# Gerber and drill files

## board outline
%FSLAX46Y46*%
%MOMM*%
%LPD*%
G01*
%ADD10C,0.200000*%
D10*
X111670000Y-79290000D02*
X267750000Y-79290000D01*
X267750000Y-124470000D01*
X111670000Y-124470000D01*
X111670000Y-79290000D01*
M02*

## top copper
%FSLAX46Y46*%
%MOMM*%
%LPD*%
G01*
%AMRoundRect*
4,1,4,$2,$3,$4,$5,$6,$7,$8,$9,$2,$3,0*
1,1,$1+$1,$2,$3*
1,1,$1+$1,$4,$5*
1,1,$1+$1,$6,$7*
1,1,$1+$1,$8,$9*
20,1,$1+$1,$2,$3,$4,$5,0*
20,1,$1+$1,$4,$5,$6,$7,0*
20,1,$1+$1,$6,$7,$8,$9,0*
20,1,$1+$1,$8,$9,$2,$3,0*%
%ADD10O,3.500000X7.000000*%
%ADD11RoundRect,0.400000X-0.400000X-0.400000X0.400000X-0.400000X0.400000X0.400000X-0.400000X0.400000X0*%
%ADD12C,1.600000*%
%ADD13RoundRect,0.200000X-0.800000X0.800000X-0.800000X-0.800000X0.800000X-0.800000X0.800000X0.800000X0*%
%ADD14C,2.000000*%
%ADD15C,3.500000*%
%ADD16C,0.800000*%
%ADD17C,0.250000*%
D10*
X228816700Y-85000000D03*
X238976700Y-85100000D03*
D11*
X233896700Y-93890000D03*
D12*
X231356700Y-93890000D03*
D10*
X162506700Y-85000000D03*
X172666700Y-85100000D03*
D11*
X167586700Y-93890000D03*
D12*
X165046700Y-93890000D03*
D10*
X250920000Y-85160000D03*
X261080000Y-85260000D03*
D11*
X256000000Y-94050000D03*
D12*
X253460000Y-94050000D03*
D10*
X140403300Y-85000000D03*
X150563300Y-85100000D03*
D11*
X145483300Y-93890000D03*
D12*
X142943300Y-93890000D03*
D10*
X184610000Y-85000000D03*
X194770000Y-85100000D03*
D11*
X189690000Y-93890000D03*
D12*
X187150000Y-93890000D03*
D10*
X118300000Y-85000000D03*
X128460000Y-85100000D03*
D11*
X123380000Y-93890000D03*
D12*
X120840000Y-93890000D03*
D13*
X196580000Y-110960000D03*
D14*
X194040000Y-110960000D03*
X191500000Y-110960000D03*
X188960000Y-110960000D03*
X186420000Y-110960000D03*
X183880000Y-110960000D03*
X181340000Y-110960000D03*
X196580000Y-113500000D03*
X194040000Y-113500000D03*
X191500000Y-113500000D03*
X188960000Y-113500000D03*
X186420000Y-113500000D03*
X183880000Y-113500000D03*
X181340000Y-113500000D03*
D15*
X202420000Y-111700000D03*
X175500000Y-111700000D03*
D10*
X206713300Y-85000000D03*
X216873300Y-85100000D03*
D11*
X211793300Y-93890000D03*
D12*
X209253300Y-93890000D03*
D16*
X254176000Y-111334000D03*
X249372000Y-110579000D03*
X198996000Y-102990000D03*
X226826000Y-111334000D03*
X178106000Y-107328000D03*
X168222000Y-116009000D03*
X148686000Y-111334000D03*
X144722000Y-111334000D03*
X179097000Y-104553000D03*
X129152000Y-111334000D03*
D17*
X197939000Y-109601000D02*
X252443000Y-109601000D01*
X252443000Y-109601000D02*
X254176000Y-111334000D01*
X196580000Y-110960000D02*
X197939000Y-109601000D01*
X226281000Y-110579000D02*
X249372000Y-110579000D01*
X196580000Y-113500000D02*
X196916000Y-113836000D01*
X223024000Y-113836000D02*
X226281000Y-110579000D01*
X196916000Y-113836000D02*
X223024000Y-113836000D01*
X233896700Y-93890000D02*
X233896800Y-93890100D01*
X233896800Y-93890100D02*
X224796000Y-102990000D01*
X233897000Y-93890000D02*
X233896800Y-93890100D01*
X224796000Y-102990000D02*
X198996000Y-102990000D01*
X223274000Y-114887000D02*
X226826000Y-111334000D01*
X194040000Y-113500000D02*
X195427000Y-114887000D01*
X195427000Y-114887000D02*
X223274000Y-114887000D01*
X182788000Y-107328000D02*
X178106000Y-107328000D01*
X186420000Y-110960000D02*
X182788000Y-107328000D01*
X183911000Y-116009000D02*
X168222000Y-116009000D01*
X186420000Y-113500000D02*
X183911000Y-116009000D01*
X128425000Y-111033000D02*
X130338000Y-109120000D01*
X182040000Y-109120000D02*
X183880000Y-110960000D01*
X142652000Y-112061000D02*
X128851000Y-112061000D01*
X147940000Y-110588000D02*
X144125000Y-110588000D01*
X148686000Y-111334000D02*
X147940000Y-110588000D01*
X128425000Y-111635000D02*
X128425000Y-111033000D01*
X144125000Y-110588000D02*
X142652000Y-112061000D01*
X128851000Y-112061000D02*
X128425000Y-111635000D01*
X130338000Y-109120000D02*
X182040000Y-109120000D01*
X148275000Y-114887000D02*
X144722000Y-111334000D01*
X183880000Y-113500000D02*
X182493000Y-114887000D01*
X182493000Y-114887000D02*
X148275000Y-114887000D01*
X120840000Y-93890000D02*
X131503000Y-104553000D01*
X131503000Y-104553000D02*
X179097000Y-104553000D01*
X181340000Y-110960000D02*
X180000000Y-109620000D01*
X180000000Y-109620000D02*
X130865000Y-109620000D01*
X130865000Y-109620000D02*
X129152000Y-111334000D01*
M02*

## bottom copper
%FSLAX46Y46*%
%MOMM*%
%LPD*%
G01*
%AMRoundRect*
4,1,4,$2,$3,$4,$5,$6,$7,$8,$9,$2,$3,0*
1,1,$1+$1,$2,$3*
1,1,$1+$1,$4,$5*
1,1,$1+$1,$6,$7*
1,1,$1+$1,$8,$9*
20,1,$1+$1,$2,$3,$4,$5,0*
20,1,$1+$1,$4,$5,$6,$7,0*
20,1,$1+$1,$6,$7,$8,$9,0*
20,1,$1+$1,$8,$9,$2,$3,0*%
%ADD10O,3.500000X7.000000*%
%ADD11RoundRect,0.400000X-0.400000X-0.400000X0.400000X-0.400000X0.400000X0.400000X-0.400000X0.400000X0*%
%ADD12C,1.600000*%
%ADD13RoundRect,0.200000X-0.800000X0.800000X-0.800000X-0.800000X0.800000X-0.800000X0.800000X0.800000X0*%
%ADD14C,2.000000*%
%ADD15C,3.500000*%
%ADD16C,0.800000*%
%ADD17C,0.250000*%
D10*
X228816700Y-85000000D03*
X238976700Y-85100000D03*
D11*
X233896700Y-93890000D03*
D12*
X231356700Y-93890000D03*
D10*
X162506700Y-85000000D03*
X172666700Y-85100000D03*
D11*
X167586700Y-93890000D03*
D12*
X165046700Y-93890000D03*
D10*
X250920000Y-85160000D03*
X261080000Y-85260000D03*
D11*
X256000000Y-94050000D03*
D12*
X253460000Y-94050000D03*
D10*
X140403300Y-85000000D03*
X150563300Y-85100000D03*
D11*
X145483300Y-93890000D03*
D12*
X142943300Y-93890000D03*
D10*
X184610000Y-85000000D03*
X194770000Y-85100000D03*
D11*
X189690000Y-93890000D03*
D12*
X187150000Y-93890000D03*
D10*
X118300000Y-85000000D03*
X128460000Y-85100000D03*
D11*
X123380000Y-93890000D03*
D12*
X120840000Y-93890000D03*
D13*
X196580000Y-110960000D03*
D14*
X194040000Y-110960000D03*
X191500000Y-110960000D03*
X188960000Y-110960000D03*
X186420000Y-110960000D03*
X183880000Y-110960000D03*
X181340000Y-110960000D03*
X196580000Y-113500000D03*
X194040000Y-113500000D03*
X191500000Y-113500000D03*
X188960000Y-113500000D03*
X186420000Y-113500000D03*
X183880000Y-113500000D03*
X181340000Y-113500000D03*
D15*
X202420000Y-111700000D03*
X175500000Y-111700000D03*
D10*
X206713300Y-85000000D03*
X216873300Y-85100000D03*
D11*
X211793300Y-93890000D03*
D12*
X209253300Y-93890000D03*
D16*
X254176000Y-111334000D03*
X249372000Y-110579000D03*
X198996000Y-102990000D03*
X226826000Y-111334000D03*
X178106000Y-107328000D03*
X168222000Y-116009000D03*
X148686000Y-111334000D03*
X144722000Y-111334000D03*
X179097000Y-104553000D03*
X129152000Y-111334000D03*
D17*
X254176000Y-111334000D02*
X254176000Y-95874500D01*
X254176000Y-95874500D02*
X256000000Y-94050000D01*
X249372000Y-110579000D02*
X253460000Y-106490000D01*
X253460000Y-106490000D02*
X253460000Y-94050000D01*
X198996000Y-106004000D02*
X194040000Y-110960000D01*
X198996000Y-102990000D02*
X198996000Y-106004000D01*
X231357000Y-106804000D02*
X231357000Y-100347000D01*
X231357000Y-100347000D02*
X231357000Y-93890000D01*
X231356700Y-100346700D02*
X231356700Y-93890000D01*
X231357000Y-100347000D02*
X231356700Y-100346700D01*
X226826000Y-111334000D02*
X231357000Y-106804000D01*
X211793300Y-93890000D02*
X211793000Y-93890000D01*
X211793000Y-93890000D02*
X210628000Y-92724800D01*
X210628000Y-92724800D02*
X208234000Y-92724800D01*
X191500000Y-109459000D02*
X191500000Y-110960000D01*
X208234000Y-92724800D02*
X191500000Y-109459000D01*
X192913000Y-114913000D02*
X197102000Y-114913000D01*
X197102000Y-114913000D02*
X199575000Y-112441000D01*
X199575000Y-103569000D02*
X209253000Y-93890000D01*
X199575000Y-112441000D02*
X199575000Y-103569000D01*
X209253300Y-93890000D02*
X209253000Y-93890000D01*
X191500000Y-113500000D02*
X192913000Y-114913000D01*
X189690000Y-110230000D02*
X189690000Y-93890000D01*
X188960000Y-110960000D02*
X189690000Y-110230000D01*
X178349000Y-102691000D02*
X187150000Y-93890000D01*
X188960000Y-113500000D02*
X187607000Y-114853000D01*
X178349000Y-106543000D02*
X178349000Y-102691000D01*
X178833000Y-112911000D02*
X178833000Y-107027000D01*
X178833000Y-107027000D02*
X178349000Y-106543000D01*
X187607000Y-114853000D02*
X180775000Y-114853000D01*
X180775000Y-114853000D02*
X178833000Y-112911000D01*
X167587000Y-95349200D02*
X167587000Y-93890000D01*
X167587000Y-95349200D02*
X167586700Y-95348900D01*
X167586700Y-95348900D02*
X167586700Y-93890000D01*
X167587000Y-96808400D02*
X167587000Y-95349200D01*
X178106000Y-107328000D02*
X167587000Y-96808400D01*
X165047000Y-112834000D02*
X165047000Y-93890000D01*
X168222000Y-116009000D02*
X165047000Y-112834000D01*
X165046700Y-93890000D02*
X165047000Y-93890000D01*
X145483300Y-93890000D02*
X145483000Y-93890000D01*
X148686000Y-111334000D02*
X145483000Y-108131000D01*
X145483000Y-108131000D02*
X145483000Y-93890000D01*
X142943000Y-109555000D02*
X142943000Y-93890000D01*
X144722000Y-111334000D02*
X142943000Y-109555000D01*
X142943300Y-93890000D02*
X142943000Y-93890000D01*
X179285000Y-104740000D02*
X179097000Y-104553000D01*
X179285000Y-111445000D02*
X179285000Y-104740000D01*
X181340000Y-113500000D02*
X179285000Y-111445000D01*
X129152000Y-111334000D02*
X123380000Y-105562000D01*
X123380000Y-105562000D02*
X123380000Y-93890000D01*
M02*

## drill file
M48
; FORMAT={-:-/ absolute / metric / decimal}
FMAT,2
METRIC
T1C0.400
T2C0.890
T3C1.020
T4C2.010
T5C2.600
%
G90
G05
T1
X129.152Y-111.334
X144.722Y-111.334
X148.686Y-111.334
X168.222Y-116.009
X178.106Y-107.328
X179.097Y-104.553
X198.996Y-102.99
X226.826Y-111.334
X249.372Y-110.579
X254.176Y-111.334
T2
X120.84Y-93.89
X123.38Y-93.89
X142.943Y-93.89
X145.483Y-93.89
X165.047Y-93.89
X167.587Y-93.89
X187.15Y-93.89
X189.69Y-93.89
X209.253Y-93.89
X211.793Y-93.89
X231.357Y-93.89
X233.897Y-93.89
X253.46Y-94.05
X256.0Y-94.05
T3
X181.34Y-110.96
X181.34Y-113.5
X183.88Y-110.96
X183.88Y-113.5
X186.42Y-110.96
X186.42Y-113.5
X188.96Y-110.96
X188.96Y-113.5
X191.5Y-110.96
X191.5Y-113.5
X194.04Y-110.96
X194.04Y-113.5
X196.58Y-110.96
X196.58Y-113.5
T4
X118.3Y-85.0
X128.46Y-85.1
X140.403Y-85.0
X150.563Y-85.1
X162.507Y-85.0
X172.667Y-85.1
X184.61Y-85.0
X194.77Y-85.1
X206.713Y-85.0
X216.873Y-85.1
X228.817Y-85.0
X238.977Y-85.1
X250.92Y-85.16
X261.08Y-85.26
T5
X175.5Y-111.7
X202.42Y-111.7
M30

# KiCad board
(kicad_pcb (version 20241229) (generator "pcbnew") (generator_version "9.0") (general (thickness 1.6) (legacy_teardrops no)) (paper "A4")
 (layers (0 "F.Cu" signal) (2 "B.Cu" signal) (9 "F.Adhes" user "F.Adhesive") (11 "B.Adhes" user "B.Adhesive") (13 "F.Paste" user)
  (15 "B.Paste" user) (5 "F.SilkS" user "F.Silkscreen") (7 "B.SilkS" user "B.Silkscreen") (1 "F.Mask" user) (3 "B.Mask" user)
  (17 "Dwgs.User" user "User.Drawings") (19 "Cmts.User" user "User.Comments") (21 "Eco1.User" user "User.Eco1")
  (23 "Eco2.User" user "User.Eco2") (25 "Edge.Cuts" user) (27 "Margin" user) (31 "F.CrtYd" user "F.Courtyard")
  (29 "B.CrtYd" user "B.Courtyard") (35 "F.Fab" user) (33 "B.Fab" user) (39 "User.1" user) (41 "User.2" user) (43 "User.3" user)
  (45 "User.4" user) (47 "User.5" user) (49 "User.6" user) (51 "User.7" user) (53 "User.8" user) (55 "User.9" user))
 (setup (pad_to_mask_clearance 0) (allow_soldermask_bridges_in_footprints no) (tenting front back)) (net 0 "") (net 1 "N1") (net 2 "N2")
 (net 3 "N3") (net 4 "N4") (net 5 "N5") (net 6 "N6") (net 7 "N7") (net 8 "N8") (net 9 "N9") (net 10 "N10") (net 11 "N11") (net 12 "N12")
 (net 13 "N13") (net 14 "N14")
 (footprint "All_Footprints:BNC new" (layer "F.Cu") (at 233.8967 93.89)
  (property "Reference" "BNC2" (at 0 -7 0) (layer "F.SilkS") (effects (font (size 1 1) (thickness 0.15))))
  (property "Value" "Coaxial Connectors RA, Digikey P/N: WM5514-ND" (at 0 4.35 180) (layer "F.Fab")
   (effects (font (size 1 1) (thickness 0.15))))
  (pad "" thru_hole oval (at -5.08 -8.89) (size 3.5 7) (drill 2.01) (layers "*.Cu" "*.Mask") (remove_unused_layers no))
  (pad "" thru_hole oval (at 5.08 -8.79) (size 3.5 7) (drill 2.01) (layers "*.Cu" "*.Mask") (remove_unused_layers no))
  (pad "1" thru_hole roundrect (at 0 0) (size 1.6 1.6) (drill 0.89) (layers "*.Cu" "*.Mask") (remove_unused_layers no)
   (roundrect_rratio 0.25) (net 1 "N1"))
  (pad "2" thru_hole circle (at -2.54 0) (size 1.6 1.6) (drill 0.89) (layers "*.Cu" "*.Mask") (remove_unused_layers no) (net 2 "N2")))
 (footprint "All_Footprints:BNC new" (layer "F.Cu") (at 167.5867 93.89)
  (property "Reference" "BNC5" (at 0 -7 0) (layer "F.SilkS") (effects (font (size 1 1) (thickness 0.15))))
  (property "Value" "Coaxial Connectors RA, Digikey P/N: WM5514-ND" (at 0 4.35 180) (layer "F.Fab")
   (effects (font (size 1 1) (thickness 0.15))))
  (pad "" thru_hole oval (at -5.08 -8.89) (size 3.5 7) (drill 2.01) (layers "*.Cu" "*.Mask") (remove_unused_layers no))
  (pad "" thru_hole oval (at 5.08 -8.79) (size 3.5 7) (drill 2.01) (layers "*.Cu" "*.Mask") (remove_unused_layers no))
  (pad "1" thru_hole roundrect (at 0 0) (size 1.6 1.6) (drill 0.89) (layers "*.Cu" "*.Mask") (remove_unused_layers no)
   (roundrect_rratio 0.25) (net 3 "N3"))
  (pad "2" thru_hole circle (at -2.54 0) (size 1.6 1.6) (drill 0.89) (layers "*.Cu" "*.Mask") (remove_unused_layers no) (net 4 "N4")))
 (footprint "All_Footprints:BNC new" (layer "F.Cu") (at 256 94.05)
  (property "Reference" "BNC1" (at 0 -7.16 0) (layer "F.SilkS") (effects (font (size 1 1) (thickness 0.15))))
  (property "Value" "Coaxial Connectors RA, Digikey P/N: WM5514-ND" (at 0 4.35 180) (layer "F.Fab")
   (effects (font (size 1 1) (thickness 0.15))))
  (pad "" thru_hole oval (at -5.08 -8.89) (size 3.5 7) (drill 2.01) (layers "*.Cu" "*.Mask") (remove_unused_layers no))
  (pad "" thru_hole oval (at 5.08 -8.79) (size 3.5 7) (drill 2.01) (layers "*.Cu" "*.Mask") (remove_unused_layers no))
  (pad "1" thru_hole roundrect (at 0 0) (size 1.6 1.6) (drill 0.89) (layers "*.Cu" "*.Mask") (remove_unused_layers no)
   (roundrect_rratio 0.25) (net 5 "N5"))
  (pad "2" thru_hole circle (at -2.54 0) (size 1.6 1.6) (drill 0.89) (layers "*.Cu" "*.Mask") (remove_unused_layers no) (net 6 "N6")))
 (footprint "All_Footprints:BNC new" (layer "F.Cu") (at 145.4833 93.89)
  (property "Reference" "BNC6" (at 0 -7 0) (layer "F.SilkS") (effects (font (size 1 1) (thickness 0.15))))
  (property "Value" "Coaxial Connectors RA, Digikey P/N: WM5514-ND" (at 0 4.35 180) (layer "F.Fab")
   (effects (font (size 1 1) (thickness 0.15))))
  (pad "" thru_hole oval (at -5.08 -8.89) (size 3.5 7) (drill 2.01) (layers "*.Cu" "*.Mask") (remove_unused_layers no))
  (pad "" thru_hole oval (at 5.08 -8.79) (size 3.5 7) (drill 2.01) (layers "*.Cu" "*.Mask") (remove_unused_layers no))
  (pad "1" thru_hole roundrect (at 0 0) (size 1.6 1.6) (drill 0.89) (layers "*.Cu" "*.Mask") (remove_unused_layers no)
   (roundrect_rratio 0.25) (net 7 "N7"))
  (pad "2" thru_hole circle (at -2.54 0) (size 1.6 1.6) (drill 0.89) (layers "*.Cu" "*.Mask") (remove_unused_layers no) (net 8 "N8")))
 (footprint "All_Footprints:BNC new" (layer "F.Cu") (at 189.69 93.89)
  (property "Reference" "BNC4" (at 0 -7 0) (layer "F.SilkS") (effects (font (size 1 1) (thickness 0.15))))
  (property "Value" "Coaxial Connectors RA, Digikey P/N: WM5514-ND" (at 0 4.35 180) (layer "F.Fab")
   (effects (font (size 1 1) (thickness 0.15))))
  (pad "" thru_hole oval (at -5.08 -8.89) (size 3.5 7) (drill 2.01) (layers "*.Cu" "*.Mask") (remove_unused_layers no))
  (pad "" thru_hole oval (at 5.08 -8.79) (size 3.5 7) (drill 2.01) (layers "*.Cu" "*.Mask") (remove_unused_layers no))
  (pad "1" thru_hole roundrect (at 0 0) (size 1.6 1.6) (drill 0.89) (layers "*.Cu" "*.Mask") (remove_unused_layers no)
   (roundrect_rratio 0.25) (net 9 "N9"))
  (pad "2" thru_hole circle (at -2.54 0) (size 1.6 1.6) (drill 0.89) (layers "*.Cu" "*.Mask") (remove_unused_layers no) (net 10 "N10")))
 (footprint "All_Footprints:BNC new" (layer "F.Cu") (at 123.38 93.89)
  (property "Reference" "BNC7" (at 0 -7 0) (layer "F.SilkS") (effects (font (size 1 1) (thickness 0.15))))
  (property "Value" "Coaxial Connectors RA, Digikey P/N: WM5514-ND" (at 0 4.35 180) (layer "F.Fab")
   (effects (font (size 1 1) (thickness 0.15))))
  (pad "" thru_hole oval (at -5.08 -8.89) (size 3.5 7) (drill 2.01) (layers "*.Cu" "*.Mask") (remove_unused_layers no))
  (pad "" thru_hole oval (at 5.08 -8.79) (size 3.5 7) (drill 2.01) (layers "*.Cu" "*.Mask") (remove_unused_layers no))
  (pad "1" thru_hole roundrect (at 0 0) (size 1.6 1.6) (drill 0.89) (layers "*.Cu" "*.Mask") (remove_unused_layers no)
   (roundrect_rratio 0.25) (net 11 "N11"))
  (pad "2" thru_hole circle (at -2.54 0) (size 1.6 1.6) (drill 0.89) (layers "*.Cu" "*.Mask") (remove_unused_layers no) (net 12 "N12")))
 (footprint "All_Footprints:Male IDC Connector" (layer "F.Cu") (at 207.42 105.85 -90)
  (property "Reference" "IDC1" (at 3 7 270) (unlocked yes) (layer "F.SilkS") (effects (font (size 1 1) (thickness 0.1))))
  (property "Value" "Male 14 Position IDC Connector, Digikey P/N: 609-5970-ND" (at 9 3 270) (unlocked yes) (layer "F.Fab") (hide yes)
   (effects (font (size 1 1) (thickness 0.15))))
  (pad "1" thru_hole roundrect (at 5.11 10.84 270) (size 2 2) (drill 1.02) (layers "*.Cu" "*.Mask") (remove_unused_layers no)
   (roundrect_rratio 0.1) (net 5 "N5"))
  (pad "2" thru_hole circle (at 5.11 13.38 270) (size 2 2) (drill 1.02) (layers "*.Cu" "*.Mask") (remove_unused_layers no) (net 1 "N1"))
  (pad "3" thru_hole circle (at 5.11 15.92 270) (size 2 2) (drill 1.02) (layers "*.Cu" "*.Mask") (remove_unused_layers no) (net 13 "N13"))
  (pad "4" thru_hole circle (at 5.11 18.46 270) (size 2 2) (drill 1.02) (layers "*.Cu" "*.Mask") (remove_unused_layers no) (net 9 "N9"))
  (pad "5" thru_hole circle (at 5.11 21 270) (size 2 2) (drill 1.02) (layers "*.Cu" "*.Mask") (remove_unused_layers no) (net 3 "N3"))
  (pad "6" thru_hole circle (at 5.11 23.54 270) (size 2 2) (drill 1.02) (layers "*.Cu" "*.Mask") (remove_unused_layers no) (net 7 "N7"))
  (pad "7" thru_hole circle (at 5.11 26.08 270) (size 2 2) (drill 1.02) (layers "*.Cu" "*.Mask") (remove_unused_layers no) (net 11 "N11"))
  (pad "8" thru_hole circle (at 7.65 10.84 270) (size 2 2) (drill 1.02) (layers "*.Cu" "*.Mask") (remove_unused_layers no) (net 6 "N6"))
  (pad "9" thru_hole circle (at 7.65 13.38 270) (size 2 2) (drill 1.02) (layers "*.Cu" "*.Mask") (remove_unused_layers no) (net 2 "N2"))
  (pad "10" thru_hole circle (at 7.65 15.92 270) (size 2 2) (drill 1.02) (layers "*.Cu" "*.Mask") (remove_unused_layers no) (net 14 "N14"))
  (pad "11" thru_hole circle (at 7.65 18.46 270) (size 2 2) (drill 1.02) (layers "*.Cu" "*.Mask") (remove_unused_layers no) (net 10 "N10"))
  (pad "12" thru_hole circle (at 7.65 21 270) (size 2 2) (drill 1.02) (layers "*.Cu" "*.Mask") (remove_unused_layers no) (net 4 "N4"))
  (pad "13" thru_hole circle (at 7.65 23.54 270) (size 2 2) (drill 1.02) (layers "*.Cu" "*.Mask") (remove_unused_layers no) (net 8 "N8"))
  (pad "14" thru_hole circle (at 7.65 26.08 270) (size 2 2) (drill 1.02) (layers "*.Cu" "*.Mask") (remove_unused_layers no) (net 12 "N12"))
  (pad "MH" thru_hole circle (at 5.85 5 270) (size 3.5 3.5) (drill 2.6) (layers "*.Cu" "*.Mask") (remove_unused_layers no))
  (pad "MH" thru_hole circle (at 5.85 31.92 270) (size 3.5 3.5) (drill 2.6) (layers "*.Cu" "*.Mask") (remove_unused_layers no)))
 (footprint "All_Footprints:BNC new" (layer "F.Cu") (at 211.7933 93.89)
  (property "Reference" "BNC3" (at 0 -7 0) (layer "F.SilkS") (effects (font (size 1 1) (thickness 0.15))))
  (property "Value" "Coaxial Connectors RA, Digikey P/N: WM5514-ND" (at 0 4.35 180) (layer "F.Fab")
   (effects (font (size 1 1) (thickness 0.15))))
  (pad "" thru_hole oval (at -5.08 -8.89) (size 3.5 7) (drill 2.01) (layers "*.Cu" "*.Mask") (remove_unused_layers no))
  (pad "" thru_hole oval (at 5.08 -8.79) (size 3.5 7) (drill 2.01) (layers "*.Cu" "*.Mask") (remove_unused_layers no))
  (pad "1" thru_hole roundrect (at 0 0) (size 1.6 1.6) (drill 0.89) (layers "*.Cu" "*.Mask") (remove_unused_layers no)
   (roundrect_rratio 0.25) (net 13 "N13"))
  (pad "2" thru_hole circle (at -2.54 0) (size 1.6 1.6) (drill 0.89) (layers "*.Cu" "*.Mask") (remove_unused_layers no) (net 14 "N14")))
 (gr_rect (start 111.67 79.29) (end 267.75 124.47) (stroke (width 0.2) (type solid)) (fill no) (layer "Edge.Cuts"))
 (segment (start 197.939 109.601) (end 252.443 109.601) (width 0.25) (layer "F.Cu") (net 5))
 (segment (start 252.443 109.601) (end 254.176 111.334) (width 0.25) (layer "F.Cu") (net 5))
 (segment (start 196.58 110.96) (end 197.939 109.601) (width 0.25) (layer "F.Cu") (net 5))
 (via (at 254.176 111.334) (size 0.8) (drill 0.4) (layers "F.Cu" "B.Cu") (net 5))
 (segment (start 254.176 111.334) (end 254.176 95.8745) (width 0.25) (layer "B.Cu") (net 5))
 (segment (start 254.176 95.8745) (end 256 94.05) (width 0.25) (layer "B.Cu") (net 5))
 (segment (start 226.281 110.579) (end 249.372 110.579) (width 0.25) (layer "F.Cu") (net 6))
 (segment (start 196.58 113.5) (end 196.916 113.836) (width 0.25) (layer "F.Cu") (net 6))
 (segment (start 223.024 113.836) (end 226.281 110.579) (width 0.25) (layer "F.Cu") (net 6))
 (segment (start 196.916 113.836) (end 223.024 113.836) (width 0.25) (layer "F.Cu") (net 6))
 (via (at 249.372 110.579) (size 0.8) (drill 0.4) (layers "F.Cu" "B.Cu") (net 6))
 (segment (start 249.372 110.579) (end 253.46 106.49) (width 0.25) (layer "B.Cu") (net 6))
 (segment (start 253.46 106.49) (end 253.46 94.05) (width 0.25) (layer "B.Cu") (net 6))
 (segment (start 233.8967 93.89) (end 233.8968 93.8901) (width 0.25) (layer "F.Cu") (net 1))
 (segment (start 233.8968 93.8901) (end 224.796 102.99) (width 0.25) (layer "F.Cu") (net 1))
 (segment (start 233.897 93.89) (end 233.8968 93.8901) (width 0.25) (layer "F.Cu") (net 1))
 (segment (start 224.796 102.99) (end 198.996 102.99) (width 0.25) (layer "F.Cu") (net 1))
 (via (at 198.996 102.99) (size 0.8) (drill 0.4) (layers "F.Cu" "B.Cu") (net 1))
 (segment (start 198.996 106.004) (end 194.04 110.96) (width 0.25) (layer "B.Cu") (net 1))
 (segment (start 198.996 102.99) (end 198.996 106.004) (width 0.25) (layer "B.Cu") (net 1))
 (segment (start 223.274 114.887) (end 226.826 111.334) (width 0.25) (layer "F.Cu") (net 2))
 (segment (start 194.04 113.5) (end 195.427 114.887) (width 0.25) (layer "F.Cu") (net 2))
 (segment (start 195.427 114.887) (end 223.274 114.887) (width 0.25) (layer "F.Cu") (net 2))
 (via (at 226.826 111.334) (size 0.8) (drill 0.4) (layers "F.Cu" "B.Cu") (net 2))
 (segment (start 231.357 106.804) (end 231.357 100.347) (width 0.25) (layer "B.Cu") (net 2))
 (segment (start 231.357 100.347) (end 231.357 93.89) (width 0.25) (layer "B.Cu") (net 2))
 (segment (start 231.3567 100.3467) (end 231.3567 93.89) (width 0.25) (layer "B.Cu") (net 2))
 (segment (start 231.357 100.347) (end 231.3567 100.3467) (width 0.25) (layer "B.Cu") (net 2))
 (segment (start 226.826 111.334) (end 231.357 106.804) (width 0.25) (layer "B.Cu") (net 2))
 (segment (start 211.7933 93.89) (end 211.793 93.89) (width 0.25) (layer "B.Cu") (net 13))
 (segment (start 211.793 93.89) (end 210.628 92.7248) (width 0.25) (layer "B.Cu") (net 13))
 (segment (start 210.628 92.7248) (end 208.234 92.7248) (width 0.25) (layer "B.Cu") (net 13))
 (segment (start 191.5 109.459) (end 191.5 110.96) (width 0.25) (layer "B.Cu") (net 13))
 (segment (start 208.234 92.7248) (end 191.5 109.459) (width 0.25) (layer "B.Cu") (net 13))
 (segment (start 192.913 114.913) (end 197.102 114.913) (width 0.25) (layer "B.Cu") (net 14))
 (segment (start 197.102 114.913) (end 199.575 112.441) (width 0.25) (layer "B.Cu") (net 14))
 (segment (start 199.575 103.569) (end 209.253 93.89) (width 0.25) (layer "B.Cu") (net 14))
 (segment (start 199.575 112.441) (end 199.575 103.569) (width 0.25) (layer "B.Cu") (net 14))
 (segment (start 209.2533 93.89) (end 209.253 93.89) (width 0.25) (layer "B.Cu") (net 14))
 (segment (start 191.5 113.5) (end 192.913 114.913) (width 0.25) (layer "B.Cu") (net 14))
 (segment (start 189.69 110.23) (end 189.69 93.89) (width 0.25) (layer "B.Cu") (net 9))
 (segment (start 188.96 110.96) (end 189.69 110.23) (width 0.25) (layer "B.Cu") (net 9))
 (segment (start 178.349 102.691) (end 187.15 93.89) (width 0.25) (layer "B.Cu") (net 10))
 (segment (start 188.96 113.5) (end 187.607 114.853) (width 0.25) (layer "B.Cu") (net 10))
 (segment (start 178.349 106.543) (end 178.349 102.691) (width 0.25) (layer "B.Cu") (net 10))
 (segment (start 178.833 112.911) (end 178.833 107.027) (width 0.25) (layer "B.Cu") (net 10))
 (segment (start 178.833 107.027) (end 178.349 106.543) (width 0.25) (layer "B.Cu") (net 10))
 (segment (start 187.607 114.853) (end 180.775 114.853) (width 0.25) (layer "B.Cu") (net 10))
 (segment (start 180.775 114.853) (end 178.833 112.911) (width 0.25) (layer "B.Cu") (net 10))
 (segment (start 182.788 107.328) (end 178.106 107.328) (width 0.25) (layer "F.Cu") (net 3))
 (segment (start 186.42 110.96) (end 182.788 107.328) (width 0.25) (layer "F.Cu") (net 3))
 (via (at 178.106 107.328) (size 0.8) (drill 0.4) (layers "F.Cu" "B.Cu") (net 3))
 (segment (start 167.587 95.3492) (end 167.587 93.89) (width 0.25) (layer "B.Cu") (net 3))
 (segment (start 167.587 95.3492) (end 167.5867 95.3489) (width 0.25) (layer "B.Cu") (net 3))
 (segment (start 167.5867 95.3489) (end 167.5867 93.89) (width 0.25) (layer "B.Cu") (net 3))
 (segment (start 167.587 96.8084) (end 167.587 95.3492) (width 0.25) (layer "B.Cu") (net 3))
 (segment (start 178.106 107.328) (end 167.587 96.8084) (width 0.25) (layer "B.Cu") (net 3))
 (segment (start 183.911 116.009) (end 168.222 116.009) (width 0.25) (layer "F.Cu") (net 4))
 (segment (start 186.42 113.5) (end 183.911 116.009) (width 0.25) (layer "F.Cu") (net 4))
 (via (at 168.222 116.009) (size 0.8) (drill 0.4) (layers "F.Cu" "B.Cu") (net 4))
 (segment (start 165.047 112.834) (end 165.047 93.89) (width 0.25) (layer "B.Cu") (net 4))
 (segment (start 168.222 116.009) (end 165.047 112.834) (width 0.25) (layer "B.Cu") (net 4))
 (segment (start 165.0467 93.89) (end 165.047 93.89) (width 0.25) (layer "B.Cu") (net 4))
 (segment (start 128.425 111.033) (end 130.338 109.12) (width 0.25) (layer "F.Cu") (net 7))
 (segment (start 182.04 109.12) (end 183.88 110.96) (width 0.25) (layer "F.Cu") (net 7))
 (segment (start 142.652 112.061) (end 128.851 112.061) (width 0.25) (layer "F.Cu") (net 7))
 (segment (start 147.94 110.588) (end 144.125 110.588) (width 0.25) (layer "F.Cu") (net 7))
 (segment (start 148.686 111.334) (end 147.94 110.588) (width 0.25) (layer "F.Cu") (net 7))
 (segment (start 128.425 111.635) (end 128.425 111.033) (width 0.25) (layer "F.Cu") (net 7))
 (segment (start 144.125 110.588) (end 142.652 112.061) (width 0.25) (layer "F.Cu") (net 7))
 (segment (start 128.851 112.061) (end 128.425 111.635) (width 0.25) (layer "F.Cu") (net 7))
 (segment (start 130.338 109.12) (end 182.04 109.12) (width 0.25) (layer "F.Cu") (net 7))
 (via (at 148.686 111.334) (size 0.8) (drill 0.4) (layers "F.Cu" "B.Cu") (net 7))
 (segment (start 145.4833 93.89) (end 145.483 93.89) (width 0.25) (layer "B.Cu") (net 7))
 (segment (start 148.686 111.334) (end 145.483 108.131) (width 0.25) (layer "B.Cu") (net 7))
 (segment (start 145.483 108.131) (end 145.483 93.89) (width 0.25) (layer "B.Cu") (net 7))
 (segment (start 148.275 114.887) (end 144.722 111.334) (width 0.25) (layer "F.Cu") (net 8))
 (segment (start 183.88 113.5) (end 182.493 114.887) (width 0.25) (layer "F.Cu") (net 8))
 (segment (start 182.493 114.887) (end 148.275 114.887) (width 0.25) (layer "F.Cu") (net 8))
 (via (at 144.722 111.334) (size 0.8) (drill 0.4) (layers "F.Cu" "B.Cu") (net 8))
 (segment (start 142.943 109.555) (end 142.943 93.89) (width 0.25) (layer "B.Cu") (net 8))
 (segment (start 144.722 111.334) (end 142.943 109.555) (width 0.25) (layer "B.Cu") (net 8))
 (segment (start 142.9433 93.89) (end 142.943 93.89) (width 0.25) (layer "B.Cu") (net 8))
 (segment (start 120.84 93.89) (end 131.503 104.553) (width 0.25) (layer "F.Cu") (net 12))
 (segment (start 131.503 104.553) (end 179.097 104.553) (width 0.25) (layer "F.Cu") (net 12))
 (via (at 179.097 104.553) (size 0.8) (drill 0.4) (layers "F.Cu" "B.Cu") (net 12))
 (segment (start 179.285 104.74) (end 179.097 104.553) (width 0.25) (layer "B.Cu") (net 12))
 (segment (start 179.285 111.445) (end 179.285 104.74) (width 0.25) (layer "B.Cu") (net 12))
 (segment (start 181.34 113.5) (end 179.285 111.445) (width 0.25) (layer "B.Cu") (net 12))
 (segment (start 181.34 110.96) (end 180 109.62) (width 0.25) (layer "F.Cu") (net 11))
 (segment (start 180 109.62) (end 130.865 109.62) (width 0.25) (layer "F.Cu") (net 11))
 (segment (start 130.865 109.62) (end 129.152 111.334) (width 0.25) (layer "F.Cu") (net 11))
 (via (at 129.152 111.334) (size 0.8) (drill 0.4) (layers "F.Cu" "B.Cu") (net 11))
 (segment (start 129.152 111.334) (end 123.38 105.562) (width 0.25) (layer "B.Cu") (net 11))
 (segment (start 123.38 105.562) (end 123.38 93.89) (width 0.25) (layer "B.Cu") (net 11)))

